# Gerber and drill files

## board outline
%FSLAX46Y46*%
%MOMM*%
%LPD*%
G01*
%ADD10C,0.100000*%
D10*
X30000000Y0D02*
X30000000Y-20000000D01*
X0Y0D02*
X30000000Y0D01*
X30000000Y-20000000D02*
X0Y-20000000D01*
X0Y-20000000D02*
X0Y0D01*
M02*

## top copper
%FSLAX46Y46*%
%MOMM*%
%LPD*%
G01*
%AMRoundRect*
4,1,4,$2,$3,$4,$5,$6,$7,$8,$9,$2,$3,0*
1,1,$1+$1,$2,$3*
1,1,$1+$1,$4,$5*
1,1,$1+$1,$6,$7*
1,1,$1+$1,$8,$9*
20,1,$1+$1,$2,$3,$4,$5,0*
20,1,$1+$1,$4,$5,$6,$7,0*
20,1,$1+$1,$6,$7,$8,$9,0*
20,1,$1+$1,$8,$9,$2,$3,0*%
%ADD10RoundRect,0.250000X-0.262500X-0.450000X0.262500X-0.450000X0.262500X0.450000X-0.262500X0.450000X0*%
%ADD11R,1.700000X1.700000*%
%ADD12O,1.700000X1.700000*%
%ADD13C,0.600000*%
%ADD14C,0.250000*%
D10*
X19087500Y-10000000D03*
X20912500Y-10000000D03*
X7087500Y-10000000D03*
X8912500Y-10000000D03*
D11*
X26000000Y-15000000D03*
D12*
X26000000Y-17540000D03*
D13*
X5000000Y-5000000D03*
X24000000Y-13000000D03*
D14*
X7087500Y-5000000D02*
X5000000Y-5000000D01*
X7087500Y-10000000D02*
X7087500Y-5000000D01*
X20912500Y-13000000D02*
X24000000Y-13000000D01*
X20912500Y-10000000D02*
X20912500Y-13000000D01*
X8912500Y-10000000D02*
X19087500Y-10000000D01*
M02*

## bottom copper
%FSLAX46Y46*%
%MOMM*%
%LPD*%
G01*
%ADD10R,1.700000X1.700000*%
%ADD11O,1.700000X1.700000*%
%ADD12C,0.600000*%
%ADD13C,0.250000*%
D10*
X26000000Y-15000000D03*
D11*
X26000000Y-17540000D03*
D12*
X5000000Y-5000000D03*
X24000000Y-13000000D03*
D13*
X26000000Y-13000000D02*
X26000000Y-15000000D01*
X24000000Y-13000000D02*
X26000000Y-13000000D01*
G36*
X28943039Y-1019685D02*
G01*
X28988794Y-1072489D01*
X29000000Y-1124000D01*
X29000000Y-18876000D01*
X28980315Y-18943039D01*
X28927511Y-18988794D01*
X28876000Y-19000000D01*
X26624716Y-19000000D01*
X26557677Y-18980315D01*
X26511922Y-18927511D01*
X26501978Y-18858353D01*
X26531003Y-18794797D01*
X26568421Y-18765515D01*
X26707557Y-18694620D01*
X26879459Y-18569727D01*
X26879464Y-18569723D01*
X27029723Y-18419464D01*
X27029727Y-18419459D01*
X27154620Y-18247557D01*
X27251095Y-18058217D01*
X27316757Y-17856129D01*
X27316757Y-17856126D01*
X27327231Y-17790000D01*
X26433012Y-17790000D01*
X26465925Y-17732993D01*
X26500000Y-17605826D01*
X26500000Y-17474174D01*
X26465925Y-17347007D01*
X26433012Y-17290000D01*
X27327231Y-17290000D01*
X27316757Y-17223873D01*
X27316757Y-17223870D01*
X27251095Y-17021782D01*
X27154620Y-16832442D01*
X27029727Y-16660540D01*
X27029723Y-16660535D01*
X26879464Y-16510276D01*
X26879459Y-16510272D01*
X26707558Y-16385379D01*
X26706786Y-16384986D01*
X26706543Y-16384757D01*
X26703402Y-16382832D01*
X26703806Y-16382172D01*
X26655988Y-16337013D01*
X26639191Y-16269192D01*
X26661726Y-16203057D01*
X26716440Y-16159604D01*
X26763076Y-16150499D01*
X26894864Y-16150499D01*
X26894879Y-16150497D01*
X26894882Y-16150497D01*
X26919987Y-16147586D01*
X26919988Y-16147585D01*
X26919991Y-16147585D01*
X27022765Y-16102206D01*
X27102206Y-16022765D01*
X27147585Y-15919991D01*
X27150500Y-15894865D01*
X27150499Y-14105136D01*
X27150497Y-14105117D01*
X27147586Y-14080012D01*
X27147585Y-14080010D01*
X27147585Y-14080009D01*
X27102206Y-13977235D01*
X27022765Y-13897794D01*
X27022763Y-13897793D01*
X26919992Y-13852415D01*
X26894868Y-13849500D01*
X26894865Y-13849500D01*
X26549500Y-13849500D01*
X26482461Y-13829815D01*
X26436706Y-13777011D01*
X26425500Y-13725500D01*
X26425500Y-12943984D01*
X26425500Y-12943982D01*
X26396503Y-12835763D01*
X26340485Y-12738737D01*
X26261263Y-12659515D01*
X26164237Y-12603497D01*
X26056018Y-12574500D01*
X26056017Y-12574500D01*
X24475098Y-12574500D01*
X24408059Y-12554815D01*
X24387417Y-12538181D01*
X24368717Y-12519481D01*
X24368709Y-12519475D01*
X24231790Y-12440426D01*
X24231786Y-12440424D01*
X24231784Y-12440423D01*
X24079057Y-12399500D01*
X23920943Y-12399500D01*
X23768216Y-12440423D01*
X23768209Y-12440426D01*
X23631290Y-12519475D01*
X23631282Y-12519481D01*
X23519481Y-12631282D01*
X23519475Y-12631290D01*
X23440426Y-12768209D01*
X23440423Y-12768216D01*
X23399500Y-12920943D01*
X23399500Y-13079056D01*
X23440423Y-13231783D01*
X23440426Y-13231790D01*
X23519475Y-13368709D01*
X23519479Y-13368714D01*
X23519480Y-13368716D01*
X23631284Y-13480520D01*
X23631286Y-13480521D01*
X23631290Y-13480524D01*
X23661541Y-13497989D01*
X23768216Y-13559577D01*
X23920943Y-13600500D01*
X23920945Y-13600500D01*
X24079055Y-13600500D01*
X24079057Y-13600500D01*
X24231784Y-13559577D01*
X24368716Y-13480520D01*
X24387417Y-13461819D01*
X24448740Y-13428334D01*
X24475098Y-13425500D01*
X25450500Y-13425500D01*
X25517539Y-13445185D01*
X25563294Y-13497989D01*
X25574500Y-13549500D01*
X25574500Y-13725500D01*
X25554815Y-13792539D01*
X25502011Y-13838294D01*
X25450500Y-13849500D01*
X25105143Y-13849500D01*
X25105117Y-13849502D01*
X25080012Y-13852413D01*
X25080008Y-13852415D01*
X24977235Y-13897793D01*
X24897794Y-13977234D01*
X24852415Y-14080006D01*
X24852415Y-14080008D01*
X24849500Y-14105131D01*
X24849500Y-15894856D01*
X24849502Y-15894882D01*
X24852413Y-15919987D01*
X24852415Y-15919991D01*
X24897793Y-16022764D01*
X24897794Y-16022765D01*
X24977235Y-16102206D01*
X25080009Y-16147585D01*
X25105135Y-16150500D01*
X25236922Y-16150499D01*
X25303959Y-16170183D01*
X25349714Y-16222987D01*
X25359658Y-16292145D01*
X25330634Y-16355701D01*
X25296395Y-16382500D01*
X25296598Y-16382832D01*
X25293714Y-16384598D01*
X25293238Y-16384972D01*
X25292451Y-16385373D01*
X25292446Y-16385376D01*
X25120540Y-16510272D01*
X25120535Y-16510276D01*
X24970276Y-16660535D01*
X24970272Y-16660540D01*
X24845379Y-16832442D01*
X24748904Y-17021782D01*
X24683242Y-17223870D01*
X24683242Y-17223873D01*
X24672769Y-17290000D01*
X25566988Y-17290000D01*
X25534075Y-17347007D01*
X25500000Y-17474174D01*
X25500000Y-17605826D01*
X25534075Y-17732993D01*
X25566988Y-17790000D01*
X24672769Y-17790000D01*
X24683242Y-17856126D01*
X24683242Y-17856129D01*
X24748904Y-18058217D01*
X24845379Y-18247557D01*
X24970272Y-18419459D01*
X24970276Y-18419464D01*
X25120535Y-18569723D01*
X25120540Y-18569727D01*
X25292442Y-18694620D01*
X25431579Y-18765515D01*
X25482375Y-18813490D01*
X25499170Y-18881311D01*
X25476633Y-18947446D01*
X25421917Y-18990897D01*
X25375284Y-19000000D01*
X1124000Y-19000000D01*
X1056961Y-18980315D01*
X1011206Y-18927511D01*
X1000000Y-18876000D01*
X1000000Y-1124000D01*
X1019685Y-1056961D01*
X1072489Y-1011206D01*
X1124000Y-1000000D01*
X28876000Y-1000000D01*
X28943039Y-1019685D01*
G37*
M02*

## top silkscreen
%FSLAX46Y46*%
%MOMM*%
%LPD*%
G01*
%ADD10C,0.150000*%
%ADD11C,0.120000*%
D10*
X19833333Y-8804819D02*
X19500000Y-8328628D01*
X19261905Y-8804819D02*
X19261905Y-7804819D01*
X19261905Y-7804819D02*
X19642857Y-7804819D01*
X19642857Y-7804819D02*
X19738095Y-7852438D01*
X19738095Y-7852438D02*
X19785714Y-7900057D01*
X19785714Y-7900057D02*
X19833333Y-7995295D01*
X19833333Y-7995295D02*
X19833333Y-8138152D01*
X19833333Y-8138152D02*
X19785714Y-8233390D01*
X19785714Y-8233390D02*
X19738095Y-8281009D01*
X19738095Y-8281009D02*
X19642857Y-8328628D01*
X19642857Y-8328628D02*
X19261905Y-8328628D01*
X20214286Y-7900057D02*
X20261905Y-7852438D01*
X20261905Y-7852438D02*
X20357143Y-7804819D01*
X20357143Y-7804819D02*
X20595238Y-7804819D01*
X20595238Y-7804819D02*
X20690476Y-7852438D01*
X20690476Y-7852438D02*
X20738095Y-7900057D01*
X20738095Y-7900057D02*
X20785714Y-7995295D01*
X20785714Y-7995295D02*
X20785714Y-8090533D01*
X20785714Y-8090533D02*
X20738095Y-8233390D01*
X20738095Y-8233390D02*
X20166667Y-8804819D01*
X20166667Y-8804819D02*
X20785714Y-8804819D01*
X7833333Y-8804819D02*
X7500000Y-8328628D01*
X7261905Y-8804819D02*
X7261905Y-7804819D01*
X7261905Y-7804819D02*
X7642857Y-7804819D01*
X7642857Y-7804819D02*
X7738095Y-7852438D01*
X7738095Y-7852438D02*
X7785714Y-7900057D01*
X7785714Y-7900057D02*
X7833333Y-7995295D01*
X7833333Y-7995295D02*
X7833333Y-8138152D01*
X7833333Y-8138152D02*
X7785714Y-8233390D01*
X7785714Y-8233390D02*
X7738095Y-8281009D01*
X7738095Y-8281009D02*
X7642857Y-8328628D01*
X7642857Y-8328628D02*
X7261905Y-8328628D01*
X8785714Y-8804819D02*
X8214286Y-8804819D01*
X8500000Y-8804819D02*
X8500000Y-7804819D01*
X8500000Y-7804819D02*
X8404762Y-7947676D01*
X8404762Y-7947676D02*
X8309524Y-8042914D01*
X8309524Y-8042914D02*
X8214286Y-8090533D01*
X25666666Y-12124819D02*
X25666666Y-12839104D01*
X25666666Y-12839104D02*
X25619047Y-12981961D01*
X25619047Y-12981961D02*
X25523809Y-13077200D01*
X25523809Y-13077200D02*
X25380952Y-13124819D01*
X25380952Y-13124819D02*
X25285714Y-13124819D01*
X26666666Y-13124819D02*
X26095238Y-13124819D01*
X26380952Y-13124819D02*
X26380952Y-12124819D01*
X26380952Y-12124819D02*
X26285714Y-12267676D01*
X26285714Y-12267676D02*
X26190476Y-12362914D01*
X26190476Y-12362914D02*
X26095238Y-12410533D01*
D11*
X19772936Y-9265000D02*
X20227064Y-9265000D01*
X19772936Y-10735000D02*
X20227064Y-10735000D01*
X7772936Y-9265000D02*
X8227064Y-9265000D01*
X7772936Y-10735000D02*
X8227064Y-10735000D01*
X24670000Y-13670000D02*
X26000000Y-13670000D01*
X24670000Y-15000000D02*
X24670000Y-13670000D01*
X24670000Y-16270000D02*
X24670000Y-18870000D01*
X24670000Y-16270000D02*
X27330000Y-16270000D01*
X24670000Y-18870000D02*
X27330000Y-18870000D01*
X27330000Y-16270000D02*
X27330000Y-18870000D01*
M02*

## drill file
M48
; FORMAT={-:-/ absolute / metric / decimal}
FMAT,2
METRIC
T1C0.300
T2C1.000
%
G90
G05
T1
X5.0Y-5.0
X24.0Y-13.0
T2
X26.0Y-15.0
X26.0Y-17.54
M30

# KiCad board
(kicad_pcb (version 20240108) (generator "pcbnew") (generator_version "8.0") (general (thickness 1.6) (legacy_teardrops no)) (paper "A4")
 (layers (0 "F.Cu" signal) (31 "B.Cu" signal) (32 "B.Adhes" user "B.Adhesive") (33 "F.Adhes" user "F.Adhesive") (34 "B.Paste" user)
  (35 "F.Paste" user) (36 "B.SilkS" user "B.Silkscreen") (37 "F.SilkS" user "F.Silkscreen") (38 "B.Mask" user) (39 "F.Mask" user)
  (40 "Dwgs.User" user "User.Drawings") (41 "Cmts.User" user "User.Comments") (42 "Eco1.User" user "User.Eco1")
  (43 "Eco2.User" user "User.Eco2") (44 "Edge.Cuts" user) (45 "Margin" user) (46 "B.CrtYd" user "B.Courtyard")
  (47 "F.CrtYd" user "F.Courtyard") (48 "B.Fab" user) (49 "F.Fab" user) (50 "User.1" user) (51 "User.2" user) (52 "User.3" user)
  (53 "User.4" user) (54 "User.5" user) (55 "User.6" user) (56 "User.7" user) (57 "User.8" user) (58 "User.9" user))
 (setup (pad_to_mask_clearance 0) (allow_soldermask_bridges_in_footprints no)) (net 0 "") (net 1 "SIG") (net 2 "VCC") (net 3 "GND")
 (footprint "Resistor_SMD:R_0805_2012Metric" (layer "F.Cu") (at 20 10)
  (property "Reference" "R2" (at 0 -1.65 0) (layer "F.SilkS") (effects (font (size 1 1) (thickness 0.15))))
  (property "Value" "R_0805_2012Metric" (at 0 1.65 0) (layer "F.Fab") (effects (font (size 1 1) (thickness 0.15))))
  (fp_line (start -0.227064 -0.735) (end 0.227064 -0.735) (stroke (width 0.12) (type solid)) (layer "F.SilkS"))
  (fp_line (start -0.227064 0.735) (end 0.227064 0.735) (stroke (width 0.12) (type solid)) (layer "F.SilkS"))
  (pad "1" smd roundrect (at -0.9125 0) (size 1.025 1.4) (layers "F.Cu" "F.Paste" "F.Mask") (roundrect_rratio 0.243902) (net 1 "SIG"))
  (pad "2" smd roundrect (at 0.9125 0) (size 1.025 1.4) (layers "F.Cu" "F.Paste" "F.Mask") (roundrect_rratio 0.243902) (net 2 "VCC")))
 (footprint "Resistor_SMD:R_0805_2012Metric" (layer "F.Cu") (at 8 10)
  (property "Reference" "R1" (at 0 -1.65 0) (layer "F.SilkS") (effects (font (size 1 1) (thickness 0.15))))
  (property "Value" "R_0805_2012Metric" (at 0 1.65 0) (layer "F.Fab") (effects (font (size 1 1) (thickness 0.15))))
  (fp_line (start -0.227064 -0.735) (end 0.227064 -0.735) (stroke (width 0.12) (type solid)) (layer "F.SilkS"))
  (fp_line (start -0.227064 0.735) (end 0.227064 0.735) (stroke (width 0.12) (type solid)) (layer "F.SilkS"))
  (pad "1" smd roundrect (at -0.9125 0) (size 1.025 1.4) (layers "F.Cu" "F.Paste" "F.Mask") (roundrect_rratio 0.243902) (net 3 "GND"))
  (pad "2" smd roundrect (at 0.9125 0) (size 1.025 1.4) (layers "F.Cu" "F.Paste" "F.Mask") (roundrect_rratio 0.243902) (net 1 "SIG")))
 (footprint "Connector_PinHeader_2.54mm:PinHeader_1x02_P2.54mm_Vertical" (layer "F.Cu") (at 26 15)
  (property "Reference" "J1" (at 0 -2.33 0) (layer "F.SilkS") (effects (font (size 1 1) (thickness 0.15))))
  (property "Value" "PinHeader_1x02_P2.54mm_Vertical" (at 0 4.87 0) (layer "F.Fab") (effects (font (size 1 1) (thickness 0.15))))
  (fp_line (start -1.33 -1.33) (end 0 -1.33) (stroke (width 0.12) (type solid)) (layer "F.SilkS"))
  (fp_line (start -1.33 0) (end -1.33 -1.33) (stroke (width 0.12) (type solid)) (layer "F.SilkS"))
  (fp_line (start -1.33 1.27) (end -1.33 3.87) (stroke (width 0.12) (type solid)) (layer "F.SilkS"))
  (fp_line (start -1.33 1.27) (end 1.33 1.27) (stroke (width 0.12) (type solid)) (layer "F.SilkS"))
  (fp_line (start -1.33 3.87) (end 1.33 3.87) (stroke (width 0.12) (type solid)) (layer "F.SilkS"))
  (fp_line (start 1.33 1.27) (end 1.33 3.87) (stroke (width 0.12) (type solid)) (layer "F.SilkS"))
  (pad "1" thru_hole rect (at 0 0) (size 1.7 1.7) (drill 1) (layers "*.Cu" "*.Mask") (remove_unused_layers no) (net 2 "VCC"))
  (pad "2" thru_hole oval (at 0 2.54) (size 1.7 1.7) (drill 1) (layers "*.Cu" "*.Mask") (remove_unused_layers no) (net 3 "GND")))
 (gr_line (start 30 0) (end 30 20) (stroke (width 0.1) (type default)) (layer "Edge.Cuts"))
 (gr_line (start 0 0) (end 30 0) (stroke (width 0.1) (type default)) (layer "Edge.Cuts"))
 (gr_line (start 30 20) (end 0 20) (stroke (width 0.1) (type default)) (layer "Edge.Cuts"))
 (gr_line (start 0 20) (end 0 0) (stroke (width 0.1) (type default)) (layer "Edge.Cuts"))
 (segment (start 7.0875 5) (end 5 5) (width 0.25) (layer "F.Cu") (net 3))
 (segment (start 7.0875 10) (end 7.0875 5) (width 0.25) (layer "F.Cu") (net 3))
 (via (at 5 5) (size 0.6) (drill 0.3) (layers "F.Cu" "B.Cu") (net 3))
 (segment (start 20.9125 13) (end 24 13) (width 0.25) (layer "F.Cu") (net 2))
 (segment (start 20.9125 10) (end 20.9125 13) (width 0.25) (layer "F.Cu") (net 2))
 (via (at 24 13) (size 0.6) (drill 0.3) (layers "F.Cu" "B.Cu") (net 2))
 (segment (start 26 13) (end 26 15) (width 0.25) (layer "B.Cu") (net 2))
 (segment (start 24 13) (end 26 13) (width 0.25) (layer "B.Cu") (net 2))
 (segment (start 8.9125 10) (end 19.0875 10) (width 0.25) (layer "F.Cu") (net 1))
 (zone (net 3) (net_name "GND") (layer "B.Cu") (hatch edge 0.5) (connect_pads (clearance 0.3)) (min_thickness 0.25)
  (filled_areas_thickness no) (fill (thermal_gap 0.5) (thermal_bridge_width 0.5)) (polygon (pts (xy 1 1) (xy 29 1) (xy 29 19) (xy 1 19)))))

